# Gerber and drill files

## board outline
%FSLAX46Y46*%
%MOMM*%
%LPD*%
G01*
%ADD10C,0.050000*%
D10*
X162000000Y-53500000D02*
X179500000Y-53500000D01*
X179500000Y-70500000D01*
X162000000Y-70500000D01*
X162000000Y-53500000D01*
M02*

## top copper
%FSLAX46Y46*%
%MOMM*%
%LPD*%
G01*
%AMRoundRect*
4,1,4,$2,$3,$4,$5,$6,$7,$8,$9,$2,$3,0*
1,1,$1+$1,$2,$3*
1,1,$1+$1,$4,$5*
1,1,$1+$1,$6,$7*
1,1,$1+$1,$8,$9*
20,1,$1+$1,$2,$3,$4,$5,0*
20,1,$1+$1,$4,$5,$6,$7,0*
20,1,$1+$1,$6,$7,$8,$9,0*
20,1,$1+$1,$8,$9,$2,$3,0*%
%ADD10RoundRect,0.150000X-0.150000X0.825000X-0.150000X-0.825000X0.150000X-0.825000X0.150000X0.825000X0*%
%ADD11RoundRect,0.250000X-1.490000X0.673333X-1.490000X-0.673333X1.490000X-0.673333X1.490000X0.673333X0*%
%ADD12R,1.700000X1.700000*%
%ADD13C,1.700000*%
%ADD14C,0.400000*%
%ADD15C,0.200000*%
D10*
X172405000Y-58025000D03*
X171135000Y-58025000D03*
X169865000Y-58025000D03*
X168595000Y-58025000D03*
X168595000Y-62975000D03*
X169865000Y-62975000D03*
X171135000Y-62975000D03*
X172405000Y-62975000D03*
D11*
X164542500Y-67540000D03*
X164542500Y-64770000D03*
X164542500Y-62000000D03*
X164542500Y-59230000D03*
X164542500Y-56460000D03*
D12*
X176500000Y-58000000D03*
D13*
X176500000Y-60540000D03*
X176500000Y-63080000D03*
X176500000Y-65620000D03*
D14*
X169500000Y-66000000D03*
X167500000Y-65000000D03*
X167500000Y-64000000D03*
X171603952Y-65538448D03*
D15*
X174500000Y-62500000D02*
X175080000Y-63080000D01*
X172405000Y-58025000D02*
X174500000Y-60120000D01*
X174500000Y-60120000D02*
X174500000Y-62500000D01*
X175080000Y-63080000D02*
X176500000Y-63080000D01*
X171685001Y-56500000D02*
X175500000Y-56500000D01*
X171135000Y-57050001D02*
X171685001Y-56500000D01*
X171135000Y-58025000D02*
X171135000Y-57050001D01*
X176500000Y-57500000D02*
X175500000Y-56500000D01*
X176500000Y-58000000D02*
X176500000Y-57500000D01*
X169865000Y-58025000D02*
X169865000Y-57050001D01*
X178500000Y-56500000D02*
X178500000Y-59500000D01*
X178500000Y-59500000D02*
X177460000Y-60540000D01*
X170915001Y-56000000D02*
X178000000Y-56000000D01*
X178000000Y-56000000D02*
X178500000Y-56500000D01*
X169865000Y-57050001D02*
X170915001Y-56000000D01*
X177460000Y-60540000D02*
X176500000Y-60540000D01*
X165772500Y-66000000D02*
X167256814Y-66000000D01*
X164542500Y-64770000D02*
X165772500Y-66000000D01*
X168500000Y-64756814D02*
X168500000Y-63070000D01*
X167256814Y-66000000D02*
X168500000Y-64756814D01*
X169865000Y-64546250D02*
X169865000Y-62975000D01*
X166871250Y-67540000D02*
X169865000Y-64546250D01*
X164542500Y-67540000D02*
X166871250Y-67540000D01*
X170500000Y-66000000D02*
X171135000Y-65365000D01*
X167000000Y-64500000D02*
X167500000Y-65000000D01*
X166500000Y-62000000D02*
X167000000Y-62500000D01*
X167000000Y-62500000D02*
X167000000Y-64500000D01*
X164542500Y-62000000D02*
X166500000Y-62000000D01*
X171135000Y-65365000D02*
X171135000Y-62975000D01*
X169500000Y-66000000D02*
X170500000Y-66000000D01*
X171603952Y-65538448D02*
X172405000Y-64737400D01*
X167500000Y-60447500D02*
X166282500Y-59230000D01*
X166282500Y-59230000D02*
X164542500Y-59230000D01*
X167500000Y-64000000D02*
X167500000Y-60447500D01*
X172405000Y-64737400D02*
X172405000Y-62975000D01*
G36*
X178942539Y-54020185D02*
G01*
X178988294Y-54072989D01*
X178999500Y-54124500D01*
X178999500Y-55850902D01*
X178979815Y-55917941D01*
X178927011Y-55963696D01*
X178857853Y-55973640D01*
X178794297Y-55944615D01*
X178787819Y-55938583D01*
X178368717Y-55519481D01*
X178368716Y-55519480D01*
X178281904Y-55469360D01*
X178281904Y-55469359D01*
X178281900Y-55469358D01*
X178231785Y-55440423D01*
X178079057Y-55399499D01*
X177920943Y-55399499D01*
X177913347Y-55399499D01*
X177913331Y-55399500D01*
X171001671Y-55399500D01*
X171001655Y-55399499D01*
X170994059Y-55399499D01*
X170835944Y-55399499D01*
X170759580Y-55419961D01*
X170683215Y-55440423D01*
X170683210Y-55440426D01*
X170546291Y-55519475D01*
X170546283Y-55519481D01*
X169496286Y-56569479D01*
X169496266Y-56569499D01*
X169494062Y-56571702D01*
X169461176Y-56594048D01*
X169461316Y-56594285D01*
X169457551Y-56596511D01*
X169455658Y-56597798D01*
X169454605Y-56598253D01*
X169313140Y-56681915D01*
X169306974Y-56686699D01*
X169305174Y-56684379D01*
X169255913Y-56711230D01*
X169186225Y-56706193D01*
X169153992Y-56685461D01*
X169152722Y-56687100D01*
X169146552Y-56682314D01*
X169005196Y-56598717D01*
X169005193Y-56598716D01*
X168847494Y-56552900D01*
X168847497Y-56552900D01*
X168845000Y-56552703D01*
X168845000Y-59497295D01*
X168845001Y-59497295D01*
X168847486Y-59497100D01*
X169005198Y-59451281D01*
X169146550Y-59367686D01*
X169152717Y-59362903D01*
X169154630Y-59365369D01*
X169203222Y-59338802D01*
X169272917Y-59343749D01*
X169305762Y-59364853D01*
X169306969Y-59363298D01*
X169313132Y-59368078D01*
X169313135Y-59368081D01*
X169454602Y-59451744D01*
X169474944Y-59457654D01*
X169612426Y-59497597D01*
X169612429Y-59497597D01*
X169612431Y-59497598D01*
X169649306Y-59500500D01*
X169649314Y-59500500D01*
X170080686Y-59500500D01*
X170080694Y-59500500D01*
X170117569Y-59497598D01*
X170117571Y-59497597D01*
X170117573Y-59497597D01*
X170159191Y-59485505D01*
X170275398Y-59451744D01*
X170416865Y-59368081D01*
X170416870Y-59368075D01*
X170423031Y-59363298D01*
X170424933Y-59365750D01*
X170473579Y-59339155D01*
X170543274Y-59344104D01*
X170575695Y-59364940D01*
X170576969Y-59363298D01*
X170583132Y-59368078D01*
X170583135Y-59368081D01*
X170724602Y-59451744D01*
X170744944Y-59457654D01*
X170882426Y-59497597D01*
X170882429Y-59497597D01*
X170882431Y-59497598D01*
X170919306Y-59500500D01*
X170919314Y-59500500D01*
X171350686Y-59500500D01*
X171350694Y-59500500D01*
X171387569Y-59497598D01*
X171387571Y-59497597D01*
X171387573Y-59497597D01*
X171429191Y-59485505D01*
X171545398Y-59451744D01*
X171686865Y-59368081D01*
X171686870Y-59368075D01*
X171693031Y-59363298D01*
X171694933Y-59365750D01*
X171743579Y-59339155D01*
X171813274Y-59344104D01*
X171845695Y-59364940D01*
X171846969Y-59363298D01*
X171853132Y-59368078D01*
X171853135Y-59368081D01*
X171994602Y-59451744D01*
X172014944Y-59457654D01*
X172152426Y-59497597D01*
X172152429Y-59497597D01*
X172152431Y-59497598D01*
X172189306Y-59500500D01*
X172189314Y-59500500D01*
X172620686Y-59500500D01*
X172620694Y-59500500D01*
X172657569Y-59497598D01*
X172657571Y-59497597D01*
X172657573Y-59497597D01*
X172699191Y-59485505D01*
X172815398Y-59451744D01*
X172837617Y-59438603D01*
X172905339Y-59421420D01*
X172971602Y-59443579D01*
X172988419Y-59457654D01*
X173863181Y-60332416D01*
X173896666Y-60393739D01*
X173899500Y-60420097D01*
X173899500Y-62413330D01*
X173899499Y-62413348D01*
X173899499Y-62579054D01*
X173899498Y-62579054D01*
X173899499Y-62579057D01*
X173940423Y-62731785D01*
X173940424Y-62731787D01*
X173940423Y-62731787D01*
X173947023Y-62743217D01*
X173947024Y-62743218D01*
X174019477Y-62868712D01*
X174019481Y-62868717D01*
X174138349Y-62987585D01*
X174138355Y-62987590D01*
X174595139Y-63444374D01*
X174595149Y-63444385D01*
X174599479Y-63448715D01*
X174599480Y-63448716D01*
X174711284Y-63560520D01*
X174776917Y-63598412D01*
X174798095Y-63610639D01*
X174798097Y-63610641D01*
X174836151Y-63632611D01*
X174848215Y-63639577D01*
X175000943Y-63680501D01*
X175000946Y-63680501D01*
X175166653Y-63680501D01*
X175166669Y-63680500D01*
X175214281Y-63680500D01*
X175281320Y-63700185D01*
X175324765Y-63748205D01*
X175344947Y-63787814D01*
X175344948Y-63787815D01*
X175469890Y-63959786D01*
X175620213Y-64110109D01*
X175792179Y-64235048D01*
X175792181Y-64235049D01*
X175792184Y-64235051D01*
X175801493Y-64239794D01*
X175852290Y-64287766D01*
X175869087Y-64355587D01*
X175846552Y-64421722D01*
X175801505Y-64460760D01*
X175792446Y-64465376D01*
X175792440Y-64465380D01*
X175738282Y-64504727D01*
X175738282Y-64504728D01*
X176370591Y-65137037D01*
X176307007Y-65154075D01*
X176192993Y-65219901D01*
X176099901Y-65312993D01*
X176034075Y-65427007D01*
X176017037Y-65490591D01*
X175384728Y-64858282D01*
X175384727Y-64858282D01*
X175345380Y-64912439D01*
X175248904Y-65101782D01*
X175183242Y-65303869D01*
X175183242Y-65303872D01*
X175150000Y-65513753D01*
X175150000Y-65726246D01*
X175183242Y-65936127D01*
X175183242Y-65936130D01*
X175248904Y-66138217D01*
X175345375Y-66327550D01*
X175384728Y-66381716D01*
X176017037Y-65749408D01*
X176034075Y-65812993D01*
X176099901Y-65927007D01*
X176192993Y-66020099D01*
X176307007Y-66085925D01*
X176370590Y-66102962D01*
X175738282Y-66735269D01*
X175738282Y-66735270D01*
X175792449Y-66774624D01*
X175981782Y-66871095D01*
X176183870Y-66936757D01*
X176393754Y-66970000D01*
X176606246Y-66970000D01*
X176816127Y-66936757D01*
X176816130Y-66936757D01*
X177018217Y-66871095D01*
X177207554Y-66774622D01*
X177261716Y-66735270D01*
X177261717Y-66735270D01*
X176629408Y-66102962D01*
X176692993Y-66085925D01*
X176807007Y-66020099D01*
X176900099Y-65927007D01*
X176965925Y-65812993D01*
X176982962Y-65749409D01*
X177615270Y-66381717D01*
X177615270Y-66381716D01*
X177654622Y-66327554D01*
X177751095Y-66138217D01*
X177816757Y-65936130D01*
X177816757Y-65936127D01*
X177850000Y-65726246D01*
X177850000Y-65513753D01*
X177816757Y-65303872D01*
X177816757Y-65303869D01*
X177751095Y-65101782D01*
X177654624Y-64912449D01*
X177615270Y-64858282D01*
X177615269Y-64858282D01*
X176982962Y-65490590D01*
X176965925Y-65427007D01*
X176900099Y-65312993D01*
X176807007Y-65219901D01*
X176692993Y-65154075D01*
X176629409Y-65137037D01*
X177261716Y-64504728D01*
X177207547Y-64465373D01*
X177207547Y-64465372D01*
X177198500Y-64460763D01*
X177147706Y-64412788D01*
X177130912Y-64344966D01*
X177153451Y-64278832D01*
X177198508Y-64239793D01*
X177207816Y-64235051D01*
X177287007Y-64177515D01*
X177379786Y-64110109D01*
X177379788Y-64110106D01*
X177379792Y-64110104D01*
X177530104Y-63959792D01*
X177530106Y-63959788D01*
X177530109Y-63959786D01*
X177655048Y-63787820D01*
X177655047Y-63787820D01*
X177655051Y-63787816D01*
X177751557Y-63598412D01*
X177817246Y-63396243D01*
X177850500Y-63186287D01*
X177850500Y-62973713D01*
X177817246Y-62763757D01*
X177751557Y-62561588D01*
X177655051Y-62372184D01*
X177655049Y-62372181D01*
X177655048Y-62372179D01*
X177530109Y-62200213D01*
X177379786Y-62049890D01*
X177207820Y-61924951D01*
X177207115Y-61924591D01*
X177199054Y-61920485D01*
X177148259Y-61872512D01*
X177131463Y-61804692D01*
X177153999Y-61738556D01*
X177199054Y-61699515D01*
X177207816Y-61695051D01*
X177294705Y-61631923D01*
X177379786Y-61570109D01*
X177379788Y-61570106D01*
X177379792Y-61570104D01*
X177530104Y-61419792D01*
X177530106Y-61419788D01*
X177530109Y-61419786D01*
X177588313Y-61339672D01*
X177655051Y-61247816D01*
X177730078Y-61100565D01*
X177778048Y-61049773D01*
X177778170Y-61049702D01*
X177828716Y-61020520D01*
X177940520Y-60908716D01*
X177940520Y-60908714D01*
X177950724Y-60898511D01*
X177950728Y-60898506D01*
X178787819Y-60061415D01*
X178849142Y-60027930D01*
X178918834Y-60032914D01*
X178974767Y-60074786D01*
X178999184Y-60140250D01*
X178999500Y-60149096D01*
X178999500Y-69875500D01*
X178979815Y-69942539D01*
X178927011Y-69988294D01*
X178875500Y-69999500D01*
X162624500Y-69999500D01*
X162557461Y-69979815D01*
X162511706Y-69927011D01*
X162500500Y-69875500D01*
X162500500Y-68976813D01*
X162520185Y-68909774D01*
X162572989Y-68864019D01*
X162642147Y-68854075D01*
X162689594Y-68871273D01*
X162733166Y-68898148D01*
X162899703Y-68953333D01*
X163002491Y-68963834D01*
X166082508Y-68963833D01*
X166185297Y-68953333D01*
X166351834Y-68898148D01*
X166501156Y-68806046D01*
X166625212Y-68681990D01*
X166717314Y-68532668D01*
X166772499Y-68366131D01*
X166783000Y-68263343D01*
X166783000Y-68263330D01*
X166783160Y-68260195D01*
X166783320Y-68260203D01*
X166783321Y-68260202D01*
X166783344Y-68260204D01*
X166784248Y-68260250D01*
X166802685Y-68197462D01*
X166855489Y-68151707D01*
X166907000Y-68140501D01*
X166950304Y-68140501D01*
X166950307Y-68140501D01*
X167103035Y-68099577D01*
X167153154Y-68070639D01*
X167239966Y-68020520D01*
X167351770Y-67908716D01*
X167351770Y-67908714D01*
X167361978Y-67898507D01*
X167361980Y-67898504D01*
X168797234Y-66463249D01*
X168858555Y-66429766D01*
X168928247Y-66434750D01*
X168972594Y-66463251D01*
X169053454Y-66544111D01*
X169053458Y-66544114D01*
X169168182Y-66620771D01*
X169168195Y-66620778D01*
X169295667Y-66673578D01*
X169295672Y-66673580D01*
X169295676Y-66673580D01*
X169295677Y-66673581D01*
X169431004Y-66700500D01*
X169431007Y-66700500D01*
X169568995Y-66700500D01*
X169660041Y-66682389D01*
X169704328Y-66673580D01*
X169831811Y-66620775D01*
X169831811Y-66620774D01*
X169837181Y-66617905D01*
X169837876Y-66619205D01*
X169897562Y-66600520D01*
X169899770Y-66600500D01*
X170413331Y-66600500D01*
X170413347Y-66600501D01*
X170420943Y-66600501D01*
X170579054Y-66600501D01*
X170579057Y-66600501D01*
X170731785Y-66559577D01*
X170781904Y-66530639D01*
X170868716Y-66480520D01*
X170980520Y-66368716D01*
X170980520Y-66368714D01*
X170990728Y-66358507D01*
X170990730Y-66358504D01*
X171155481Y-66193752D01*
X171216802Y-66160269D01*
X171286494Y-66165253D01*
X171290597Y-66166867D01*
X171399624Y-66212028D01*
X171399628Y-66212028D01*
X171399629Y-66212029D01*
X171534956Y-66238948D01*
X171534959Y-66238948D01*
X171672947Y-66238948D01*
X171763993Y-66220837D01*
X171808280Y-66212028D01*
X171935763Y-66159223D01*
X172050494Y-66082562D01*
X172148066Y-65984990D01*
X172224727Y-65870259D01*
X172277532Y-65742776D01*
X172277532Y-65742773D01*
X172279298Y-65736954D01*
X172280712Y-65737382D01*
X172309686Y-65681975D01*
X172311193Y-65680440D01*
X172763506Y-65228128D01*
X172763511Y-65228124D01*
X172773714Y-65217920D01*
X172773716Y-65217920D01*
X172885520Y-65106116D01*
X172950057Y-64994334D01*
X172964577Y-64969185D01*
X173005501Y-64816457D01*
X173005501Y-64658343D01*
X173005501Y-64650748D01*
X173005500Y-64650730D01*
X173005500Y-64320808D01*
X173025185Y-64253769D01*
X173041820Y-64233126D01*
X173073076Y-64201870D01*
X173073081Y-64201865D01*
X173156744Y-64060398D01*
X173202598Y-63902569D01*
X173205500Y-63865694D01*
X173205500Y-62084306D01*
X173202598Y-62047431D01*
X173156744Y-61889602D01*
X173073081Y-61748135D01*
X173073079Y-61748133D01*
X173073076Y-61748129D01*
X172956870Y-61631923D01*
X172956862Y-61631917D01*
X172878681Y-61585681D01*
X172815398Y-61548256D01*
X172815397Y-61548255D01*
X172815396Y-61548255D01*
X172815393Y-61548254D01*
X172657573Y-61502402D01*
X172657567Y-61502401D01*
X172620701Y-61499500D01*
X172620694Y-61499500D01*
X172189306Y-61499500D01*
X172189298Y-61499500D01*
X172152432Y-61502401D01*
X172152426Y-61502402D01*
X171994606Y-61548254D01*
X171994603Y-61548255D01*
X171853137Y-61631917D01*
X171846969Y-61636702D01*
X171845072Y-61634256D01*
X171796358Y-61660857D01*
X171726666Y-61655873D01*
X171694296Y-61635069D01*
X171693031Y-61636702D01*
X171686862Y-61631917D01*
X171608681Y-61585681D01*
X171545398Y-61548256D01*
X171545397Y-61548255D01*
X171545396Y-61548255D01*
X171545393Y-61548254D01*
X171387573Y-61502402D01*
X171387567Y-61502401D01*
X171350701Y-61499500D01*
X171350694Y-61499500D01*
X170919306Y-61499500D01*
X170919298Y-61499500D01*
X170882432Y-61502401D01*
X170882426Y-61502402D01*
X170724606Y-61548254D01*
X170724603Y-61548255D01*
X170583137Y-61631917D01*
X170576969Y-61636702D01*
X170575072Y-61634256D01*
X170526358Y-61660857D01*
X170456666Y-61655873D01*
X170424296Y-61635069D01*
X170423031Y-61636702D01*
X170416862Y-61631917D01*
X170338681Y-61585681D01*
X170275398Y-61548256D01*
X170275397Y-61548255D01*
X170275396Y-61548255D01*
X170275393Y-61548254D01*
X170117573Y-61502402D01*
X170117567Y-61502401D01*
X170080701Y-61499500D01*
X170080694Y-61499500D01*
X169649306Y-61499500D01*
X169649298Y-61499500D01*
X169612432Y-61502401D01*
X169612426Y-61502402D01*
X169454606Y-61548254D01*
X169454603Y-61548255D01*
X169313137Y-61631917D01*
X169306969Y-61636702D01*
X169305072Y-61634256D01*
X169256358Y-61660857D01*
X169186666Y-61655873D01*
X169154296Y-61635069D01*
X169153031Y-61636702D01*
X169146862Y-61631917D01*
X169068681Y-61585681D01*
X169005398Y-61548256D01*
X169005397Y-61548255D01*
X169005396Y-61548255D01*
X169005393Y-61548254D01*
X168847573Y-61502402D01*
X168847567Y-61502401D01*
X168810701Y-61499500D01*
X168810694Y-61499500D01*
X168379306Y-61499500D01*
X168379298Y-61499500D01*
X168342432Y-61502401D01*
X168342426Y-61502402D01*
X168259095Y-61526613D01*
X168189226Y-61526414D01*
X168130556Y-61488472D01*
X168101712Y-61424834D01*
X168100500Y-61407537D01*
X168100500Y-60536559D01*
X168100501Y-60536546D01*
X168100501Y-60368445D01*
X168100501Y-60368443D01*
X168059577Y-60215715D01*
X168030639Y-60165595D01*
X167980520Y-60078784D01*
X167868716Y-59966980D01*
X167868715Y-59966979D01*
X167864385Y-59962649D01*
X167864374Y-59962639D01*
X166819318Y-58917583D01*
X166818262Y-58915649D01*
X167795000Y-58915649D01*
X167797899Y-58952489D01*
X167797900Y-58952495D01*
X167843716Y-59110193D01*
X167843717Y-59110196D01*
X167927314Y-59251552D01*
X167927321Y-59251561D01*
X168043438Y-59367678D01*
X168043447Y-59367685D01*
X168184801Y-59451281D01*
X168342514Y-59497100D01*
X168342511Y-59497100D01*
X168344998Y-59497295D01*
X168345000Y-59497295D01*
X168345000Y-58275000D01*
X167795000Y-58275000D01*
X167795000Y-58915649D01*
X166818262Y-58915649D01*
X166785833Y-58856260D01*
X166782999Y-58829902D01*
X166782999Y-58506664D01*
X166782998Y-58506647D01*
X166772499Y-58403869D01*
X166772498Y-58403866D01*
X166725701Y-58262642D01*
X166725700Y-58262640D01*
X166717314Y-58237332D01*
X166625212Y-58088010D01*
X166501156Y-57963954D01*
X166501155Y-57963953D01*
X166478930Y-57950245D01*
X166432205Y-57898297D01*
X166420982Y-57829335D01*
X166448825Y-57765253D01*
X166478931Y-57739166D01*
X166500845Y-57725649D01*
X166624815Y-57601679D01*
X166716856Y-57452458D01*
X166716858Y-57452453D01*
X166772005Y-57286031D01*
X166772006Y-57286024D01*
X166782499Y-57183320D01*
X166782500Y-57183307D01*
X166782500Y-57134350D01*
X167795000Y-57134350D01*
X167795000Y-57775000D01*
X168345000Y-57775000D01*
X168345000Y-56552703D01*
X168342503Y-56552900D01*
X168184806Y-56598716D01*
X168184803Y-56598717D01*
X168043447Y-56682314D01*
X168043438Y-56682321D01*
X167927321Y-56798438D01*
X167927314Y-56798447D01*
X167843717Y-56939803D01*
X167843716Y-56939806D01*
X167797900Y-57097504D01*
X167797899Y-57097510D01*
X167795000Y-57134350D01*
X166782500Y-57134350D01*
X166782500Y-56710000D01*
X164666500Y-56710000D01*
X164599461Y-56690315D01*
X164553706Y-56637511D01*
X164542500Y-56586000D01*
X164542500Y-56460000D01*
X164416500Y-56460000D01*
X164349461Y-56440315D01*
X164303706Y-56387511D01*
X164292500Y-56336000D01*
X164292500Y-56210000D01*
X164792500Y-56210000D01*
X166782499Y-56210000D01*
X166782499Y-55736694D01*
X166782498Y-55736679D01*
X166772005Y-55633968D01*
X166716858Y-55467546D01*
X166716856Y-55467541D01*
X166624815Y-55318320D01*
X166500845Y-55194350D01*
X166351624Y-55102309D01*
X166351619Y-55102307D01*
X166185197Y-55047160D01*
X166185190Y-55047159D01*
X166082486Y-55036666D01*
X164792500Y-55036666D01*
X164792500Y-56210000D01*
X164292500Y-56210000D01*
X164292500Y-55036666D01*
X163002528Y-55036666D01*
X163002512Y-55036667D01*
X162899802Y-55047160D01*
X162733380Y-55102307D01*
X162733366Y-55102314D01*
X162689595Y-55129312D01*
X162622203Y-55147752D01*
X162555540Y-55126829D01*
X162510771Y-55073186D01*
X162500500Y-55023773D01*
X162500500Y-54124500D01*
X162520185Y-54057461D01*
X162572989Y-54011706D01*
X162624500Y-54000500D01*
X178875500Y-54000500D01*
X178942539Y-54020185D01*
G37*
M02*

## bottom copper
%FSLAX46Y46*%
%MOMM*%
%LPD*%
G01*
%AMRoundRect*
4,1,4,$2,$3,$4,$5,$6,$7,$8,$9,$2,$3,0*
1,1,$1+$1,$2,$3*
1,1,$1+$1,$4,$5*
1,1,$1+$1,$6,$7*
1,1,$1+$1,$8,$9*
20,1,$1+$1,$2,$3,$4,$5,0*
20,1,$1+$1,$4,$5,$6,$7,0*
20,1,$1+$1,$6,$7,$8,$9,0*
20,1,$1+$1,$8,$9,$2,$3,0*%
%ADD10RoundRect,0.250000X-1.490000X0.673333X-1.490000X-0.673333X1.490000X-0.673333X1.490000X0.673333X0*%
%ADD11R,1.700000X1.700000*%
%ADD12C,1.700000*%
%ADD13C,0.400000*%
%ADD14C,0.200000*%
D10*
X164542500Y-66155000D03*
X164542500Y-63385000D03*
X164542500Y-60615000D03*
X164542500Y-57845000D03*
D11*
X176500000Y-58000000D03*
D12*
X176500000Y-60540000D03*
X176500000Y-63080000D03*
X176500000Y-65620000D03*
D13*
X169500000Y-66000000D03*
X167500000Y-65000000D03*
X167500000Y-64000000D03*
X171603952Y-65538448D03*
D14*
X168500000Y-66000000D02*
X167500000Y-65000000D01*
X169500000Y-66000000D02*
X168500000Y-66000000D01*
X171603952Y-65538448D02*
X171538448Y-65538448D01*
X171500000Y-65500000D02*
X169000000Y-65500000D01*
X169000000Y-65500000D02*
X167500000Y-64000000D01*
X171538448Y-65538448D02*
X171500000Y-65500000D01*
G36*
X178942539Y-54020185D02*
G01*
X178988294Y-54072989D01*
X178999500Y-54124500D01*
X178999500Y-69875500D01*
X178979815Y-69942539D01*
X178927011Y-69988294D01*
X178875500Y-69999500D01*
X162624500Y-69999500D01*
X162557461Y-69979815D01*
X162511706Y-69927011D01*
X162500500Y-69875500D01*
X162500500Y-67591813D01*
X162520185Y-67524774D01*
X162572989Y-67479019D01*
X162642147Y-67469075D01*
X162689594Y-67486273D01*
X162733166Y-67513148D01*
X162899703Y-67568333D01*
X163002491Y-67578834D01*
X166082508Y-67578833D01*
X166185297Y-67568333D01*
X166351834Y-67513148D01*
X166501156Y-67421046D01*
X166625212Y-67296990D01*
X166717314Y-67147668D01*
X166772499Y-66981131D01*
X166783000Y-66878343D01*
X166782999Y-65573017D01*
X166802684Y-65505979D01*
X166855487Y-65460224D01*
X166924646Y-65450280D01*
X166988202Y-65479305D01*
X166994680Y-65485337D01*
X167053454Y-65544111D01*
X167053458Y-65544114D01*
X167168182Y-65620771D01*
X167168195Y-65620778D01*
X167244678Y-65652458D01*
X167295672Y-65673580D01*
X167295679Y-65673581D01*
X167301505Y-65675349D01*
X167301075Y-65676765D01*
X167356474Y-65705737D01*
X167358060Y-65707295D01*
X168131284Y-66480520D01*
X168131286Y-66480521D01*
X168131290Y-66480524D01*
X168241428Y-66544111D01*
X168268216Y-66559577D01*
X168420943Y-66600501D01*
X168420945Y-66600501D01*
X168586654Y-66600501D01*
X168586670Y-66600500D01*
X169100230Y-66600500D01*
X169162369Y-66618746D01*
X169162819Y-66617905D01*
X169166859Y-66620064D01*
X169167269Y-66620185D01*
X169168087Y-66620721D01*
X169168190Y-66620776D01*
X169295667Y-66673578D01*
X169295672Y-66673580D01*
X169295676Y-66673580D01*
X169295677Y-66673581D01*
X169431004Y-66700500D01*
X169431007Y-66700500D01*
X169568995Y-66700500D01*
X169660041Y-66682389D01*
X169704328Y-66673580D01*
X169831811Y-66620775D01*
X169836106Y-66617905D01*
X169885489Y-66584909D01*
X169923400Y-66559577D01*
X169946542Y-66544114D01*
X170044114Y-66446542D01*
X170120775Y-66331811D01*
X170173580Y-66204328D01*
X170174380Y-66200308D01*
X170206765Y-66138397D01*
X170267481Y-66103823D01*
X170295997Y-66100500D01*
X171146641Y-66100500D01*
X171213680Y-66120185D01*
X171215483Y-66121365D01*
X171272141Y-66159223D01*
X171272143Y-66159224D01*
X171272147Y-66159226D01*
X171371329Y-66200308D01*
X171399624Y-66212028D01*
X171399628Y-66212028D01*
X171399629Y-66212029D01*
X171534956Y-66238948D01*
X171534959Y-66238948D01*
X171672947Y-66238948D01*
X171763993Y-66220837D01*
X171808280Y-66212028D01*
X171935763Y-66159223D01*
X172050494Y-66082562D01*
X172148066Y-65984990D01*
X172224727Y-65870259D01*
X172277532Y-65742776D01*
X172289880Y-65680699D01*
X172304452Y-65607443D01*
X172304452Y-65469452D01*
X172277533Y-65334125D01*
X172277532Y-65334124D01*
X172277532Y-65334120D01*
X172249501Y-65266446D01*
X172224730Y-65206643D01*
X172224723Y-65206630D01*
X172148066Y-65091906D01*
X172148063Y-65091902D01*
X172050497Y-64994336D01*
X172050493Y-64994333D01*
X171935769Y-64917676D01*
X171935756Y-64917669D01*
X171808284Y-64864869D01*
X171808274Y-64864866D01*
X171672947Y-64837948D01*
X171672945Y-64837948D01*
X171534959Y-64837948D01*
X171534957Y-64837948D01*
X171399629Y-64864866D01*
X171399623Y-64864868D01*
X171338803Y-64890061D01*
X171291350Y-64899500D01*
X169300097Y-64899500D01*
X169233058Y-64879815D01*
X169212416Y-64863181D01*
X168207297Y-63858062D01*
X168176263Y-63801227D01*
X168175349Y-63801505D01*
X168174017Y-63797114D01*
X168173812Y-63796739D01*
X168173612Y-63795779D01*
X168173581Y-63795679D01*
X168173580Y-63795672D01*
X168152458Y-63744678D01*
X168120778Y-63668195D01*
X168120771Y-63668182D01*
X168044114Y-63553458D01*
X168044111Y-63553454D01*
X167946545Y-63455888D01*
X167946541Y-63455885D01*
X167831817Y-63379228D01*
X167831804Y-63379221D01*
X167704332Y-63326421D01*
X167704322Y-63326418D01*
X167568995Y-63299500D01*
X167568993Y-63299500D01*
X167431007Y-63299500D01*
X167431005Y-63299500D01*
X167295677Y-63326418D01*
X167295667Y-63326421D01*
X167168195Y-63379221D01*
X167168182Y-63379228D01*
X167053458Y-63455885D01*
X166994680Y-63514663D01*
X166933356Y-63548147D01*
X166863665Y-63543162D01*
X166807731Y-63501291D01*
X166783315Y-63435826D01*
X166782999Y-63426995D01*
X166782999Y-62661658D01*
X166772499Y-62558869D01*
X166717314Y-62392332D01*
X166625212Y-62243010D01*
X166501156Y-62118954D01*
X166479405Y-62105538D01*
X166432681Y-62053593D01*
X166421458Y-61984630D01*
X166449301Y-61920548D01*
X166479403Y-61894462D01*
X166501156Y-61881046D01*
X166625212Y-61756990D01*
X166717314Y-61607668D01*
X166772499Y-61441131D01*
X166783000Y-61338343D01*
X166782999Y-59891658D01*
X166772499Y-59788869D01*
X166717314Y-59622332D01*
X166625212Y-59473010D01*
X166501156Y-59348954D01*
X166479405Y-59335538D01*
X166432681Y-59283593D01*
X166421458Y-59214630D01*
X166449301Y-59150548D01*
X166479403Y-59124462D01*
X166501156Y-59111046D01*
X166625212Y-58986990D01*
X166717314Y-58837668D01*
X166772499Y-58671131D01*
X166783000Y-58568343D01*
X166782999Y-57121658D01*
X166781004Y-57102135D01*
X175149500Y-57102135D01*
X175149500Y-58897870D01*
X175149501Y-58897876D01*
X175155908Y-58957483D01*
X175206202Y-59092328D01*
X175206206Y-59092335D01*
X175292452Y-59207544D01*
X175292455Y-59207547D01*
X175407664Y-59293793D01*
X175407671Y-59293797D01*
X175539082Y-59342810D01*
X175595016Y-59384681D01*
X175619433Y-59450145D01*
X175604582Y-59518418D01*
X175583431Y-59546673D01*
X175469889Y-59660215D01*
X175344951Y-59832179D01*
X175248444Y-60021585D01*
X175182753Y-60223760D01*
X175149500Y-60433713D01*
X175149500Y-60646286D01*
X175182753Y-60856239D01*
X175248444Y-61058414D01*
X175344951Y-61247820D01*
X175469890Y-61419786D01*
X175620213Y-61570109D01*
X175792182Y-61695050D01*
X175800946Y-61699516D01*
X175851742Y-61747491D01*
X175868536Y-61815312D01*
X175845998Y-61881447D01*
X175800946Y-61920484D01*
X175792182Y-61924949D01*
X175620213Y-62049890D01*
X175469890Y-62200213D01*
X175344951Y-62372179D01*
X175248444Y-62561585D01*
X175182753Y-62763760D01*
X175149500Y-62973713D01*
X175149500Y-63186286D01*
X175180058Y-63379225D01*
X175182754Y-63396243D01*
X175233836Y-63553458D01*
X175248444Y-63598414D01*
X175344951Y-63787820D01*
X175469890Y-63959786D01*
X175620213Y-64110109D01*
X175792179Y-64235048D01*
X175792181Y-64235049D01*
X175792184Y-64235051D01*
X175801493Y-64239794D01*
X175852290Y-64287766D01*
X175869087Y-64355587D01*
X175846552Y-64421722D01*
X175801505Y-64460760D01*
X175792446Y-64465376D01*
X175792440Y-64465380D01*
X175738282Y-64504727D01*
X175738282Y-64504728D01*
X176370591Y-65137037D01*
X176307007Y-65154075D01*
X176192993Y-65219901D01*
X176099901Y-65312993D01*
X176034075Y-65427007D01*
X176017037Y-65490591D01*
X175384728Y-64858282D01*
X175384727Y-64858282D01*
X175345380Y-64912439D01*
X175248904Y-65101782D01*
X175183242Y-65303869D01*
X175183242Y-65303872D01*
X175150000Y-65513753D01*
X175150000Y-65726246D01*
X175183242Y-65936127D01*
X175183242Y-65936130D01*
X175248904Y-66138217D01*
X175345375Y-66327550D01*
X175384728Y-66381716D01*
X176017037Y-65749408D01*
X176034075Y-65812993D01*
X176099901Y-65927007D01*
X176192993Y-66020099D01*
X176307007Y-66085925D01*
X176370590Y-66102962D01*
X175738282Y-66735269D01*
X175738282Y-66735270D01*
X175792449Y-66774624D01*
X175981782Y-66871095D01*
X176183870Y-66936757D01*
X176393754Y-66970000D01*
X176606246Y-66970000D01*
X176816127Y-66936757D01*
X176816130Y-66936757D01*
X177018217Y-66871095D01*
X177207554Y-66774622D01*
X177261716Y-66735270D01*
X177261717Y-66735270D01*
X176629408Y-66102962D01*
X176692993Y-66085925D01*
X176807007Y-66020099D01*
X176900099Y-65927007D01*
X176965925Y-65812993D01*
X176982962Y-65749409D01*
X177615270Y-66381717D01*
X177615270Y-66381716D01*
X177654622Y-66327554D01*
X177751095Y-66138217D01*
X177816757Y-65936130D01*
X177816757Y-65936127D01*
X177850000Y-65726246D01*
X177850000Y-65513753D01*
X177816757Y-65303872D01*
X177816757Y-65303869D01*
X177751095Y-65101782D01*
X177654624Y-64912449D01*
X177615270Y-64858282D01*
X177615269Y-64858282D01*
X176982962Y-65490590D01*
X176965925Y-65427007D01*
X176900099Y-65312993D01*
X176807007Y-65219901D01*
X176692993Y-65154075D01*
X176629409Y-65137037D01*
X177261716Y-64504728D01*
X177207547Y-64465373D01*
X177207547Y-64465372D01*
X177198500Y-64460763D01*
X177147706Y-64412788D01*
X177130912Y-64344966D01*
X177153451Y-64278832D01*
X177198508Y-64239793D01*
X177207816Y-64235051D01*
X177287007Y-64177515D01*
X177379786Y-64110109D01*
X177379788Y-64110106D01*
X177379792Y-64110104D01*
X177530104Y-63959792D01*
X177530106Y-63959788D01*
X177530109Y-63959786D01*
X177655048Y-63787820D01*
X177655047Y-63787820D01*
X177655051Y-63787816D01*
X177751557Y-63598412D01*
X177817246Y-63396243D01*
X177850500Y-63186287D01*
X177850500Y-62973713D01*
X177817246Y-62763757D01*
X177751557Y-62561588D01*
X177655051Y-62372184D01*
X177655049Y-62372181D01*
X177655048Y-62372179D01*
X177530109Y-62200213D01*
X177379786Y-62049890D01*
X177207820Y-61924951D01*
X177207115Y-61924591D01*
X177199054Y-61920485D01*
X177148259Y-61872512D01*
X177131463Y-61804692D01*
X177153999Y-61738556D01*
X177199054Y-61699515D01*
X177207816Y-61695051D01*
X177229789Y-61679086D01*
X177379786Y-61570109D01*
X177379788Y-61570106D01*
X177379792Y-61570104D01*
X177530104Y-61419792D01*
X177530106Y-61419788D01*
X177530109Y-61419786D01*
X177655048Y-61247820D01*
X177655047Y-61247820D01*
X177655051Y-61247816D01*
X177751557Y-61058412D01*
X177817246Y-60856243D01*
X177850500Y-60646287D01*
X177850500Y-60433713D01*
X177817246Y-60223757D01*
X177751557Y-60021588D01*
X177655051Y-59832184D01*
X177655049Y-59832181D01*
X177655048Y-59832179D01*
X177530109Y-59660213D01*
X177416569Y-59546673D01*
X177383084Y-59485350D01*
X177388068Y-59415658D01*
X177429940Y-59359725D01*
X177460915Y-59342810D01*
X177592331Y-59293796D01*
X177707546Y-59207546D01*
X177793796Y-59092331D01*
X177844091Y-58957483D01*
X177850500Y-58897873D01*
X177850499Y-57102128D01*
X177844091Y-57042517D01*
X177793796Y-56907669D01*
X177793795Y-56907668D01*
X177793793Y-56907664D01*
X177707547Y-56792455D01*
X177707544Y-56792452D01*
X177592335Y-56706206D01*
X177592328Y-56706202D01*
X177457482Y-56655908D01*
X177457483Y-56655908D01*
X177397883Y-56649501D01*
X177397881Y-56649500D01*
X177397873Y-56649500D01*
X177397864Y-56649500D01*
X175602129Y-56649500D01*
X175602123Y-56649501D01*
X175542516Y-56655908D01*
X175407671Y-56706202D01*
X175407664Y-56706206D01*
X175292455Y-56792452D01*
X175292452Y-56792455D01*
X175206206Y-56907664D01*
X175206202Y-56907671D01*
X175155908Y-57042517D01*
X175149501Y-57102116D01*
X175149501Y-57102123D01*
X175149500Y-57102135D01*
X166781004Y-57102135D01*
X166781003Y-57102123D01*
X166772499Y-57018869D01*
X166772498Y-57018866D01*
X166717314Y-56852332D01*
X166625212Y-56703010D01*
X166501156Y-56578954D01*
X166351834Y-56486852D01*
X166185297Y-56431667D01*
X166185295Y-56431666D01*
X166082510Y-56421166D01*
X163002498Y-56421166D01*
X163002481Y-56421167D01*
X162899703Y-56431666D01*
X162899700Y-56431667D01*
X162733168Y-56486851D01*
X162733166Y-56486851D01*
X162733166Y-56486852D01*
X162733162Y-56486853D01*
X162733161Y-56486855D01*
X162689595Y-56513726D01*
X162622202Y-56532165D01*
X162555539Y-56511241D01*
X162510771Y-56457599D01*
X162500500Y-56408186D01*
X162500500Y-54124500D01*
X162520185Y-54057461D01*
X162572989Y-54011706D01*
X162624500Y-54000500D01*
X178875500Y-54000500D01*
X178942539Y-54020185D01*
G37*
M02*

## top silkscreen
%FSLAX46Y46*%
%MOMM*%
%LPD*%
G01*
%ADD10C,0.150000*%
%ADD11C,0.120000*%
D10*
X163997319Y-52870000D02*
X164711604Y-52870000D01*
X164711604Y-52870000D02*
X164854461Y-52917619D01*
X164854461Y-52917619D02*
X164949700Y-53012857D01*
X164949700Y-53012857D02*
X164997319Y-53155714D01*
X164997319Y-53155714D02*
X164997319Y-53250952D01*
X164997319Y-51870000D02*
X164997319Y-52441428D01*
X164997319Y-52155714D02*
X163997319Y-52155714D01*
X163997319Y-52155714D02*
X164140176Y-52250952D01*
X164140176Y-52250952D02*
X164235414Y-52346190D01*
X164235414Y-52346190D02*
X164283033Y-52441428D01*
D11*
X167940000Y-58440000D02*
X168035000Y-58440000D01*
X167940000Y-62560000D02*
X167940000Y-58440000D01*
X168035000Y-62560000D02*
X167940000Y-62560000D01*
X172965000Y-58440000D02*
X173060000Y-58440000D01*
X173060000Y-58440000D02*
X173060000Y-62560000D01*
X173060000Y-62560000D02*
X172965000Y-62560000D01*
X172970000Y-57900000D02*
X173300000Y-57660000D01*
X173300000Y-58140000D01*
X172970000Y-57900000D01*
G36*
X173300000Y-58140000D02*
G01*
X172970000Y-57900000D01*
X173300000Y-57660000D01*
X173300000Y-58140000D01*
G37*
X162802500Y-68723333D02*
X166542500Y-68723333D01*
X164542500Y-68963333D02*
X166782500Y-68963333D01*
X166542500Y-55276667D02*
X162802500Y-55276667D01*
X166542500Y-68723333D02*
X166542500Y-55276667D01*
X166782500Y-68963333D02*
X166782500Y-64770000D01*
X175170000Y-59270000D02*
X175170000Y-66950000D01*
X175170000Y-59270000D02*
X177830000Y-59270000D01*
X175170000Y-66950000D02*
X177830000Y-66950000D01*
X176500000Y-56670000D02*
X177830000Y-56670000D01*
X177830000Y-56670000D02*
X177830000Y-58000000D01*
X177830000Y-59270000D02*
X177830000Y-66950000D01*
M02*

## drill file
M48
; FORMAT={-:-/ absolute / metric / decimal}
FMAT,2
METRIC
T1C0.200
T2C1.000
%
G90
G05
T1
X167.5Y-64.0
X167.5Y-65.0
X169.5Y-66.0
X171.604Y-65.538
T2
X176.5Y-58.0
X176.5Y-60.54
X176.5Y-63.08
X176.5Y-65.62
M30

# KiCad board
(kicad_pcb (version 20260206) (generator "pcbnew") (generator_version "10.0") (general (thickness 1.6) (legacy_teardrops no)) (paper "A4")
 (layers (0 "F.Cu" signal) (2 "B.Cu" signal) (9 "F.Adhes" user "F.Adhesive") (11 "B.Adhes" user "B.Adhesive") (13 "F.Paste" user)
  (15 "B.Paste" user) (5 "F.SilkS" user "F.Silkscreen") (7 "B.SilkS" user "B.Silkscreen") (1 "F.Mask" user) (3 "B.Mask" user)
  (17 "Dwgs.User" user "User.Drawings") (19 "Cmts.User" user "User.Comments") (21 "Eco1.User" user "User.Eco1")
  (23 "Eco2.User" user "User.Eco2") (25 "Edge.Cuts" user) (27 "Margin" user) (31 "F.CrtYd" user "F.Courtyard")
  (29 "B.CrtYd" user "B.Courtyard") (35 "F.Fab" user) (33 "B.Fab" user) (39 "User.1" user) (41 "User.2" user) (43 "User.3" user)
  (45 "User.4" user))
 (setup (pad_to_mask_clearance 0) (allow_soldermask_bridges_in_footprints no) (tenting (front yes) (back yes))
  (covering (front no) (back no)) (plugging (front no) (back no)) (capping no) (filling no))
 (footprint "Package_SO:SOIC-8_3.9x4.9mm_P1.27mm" (layer "F.Cu") (at 170.5 60.5 -90)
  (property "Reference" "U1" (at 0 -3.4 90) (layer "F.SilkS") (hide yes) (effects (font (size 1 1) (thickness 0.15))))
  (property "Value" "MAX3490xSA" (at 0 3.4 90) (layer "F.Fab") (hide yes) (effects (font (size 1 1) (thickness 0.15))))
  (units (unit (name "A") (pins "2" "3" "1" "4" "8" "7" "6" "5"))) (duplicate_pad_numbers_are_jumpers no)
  (fp_line (start -2.06 2.56) (end -2.06 2.465) (stroke (width 0.12) (type solid)) (layer "F.SilkS"))
  (fp_line (start 2.06 2.56) (end -2.06 2.56) (stroke (width 0.12) (type solid)) (layer "F.SilkS"))
  (fp_line (start 2.06 2.465) (end 2.06 2.56) (stroke (width 0.12) (type solid)) (layer "F.SilkS"))
  (fp_line (start -2.06 -2.465) (end -2.06 -2.56) (stroke (width 0.12) (type solid)) (layer "F.SilkS"))
  (fp_line (start -2.06 -2.56) (end 2.06 -2.56) (stroke (width 0.12) (type solid)) (layer "F.SilkS"))
  (fp_line (start 2.06 -2.56) (end 2.06 -2.465) (stroke (width 0.12) (type solid)) (layer "F.SilkS"))
  (fp_poly (pts (xy -2.6 -2.47) (xy -2.84 -2.8) (xy -2.36 -2.8)) (stroke (width 0.12) (type solid)) (fill yes) (layer "F.SilkS"))
  (pad "1" smd roundrect (at -2.475 -1.905 270) (size 1.95 0.6) (layers "F.Cu" "F.Mask" "F.Paste") (roundrect_rratio 0.25) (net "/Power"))
  (pad "2" smd roundrect (at -2.475 -0.635 270) (size 1.95 0.6) (layers "F.Cu" "F.Mask" "F.Paste") (roundrect_rratio 0.25) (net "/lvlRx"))
  (pad "3" smd roundrect (at -2.475 0.635 270) (size 1.95 0.6) (layers "F.Cu" "F.Mask" "F.Paste") (roundrect_rratio 0.25) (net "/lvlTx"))
  (pad "4" smd roundrect (at -2.475 1.905 270) (size 1.95 0.6) (layers "F.Cu" "F.Mask" "F.Paste") (roundrect_rratio 0.25) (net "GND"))
  (pad "5" smd roundrect (at 2.475 1.905 270) (size 1.95 0.6) (layers "F.Cu" "F.Mask" "F.Paste") (roundrect_rratio 0.25) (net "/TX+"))
  (pad "6" smd roundrect (at 2.475 0.635 270) (size 1.95 0.6) (layers "F.Cu" "F.Mask" "F.Paste") (roundrect_rratio 0.25) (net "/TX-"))
  (pad "7" smd roundrect (at 2.475 -0.635 270) (size 1.95 0.6) (layers "F.Cu" "F.Mask" "F.Paste") (roundrect_rratio 0.25) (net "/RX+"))
  (pad "8" smd roundrect (at 2.475 -1.905 270) (size 1.95 0.6) (layers "F.Cu" "F.Mask" "F.Paste") (roundrect_rratio 0.25) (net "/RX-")))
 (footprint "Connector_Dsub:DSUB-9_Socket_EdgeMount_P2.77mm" (layer "F.Cu") (at 164.5425 62 -90)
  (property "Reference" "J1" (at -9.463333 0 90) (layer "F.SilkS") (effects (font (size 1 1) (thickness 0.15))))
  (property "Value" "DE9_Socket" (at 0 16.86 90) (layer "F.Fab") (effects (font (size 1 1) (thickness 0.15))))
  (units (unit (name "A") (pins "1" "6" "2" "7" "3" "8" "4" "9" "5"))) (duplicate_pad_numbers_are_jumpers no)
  (fp_line (start 6.723333 1.74) (end 6.723333 -2) (stroke (width 0.12) (type solid)) (layer "F.SilkS"))
  (fp_line (start 6.963333 0) (end 6.963333 -2.24) (stroke (width 0.12) (type solid)) (layer "F.SilkS"))
  (fp_line (start -6.723333 -2) (end -6.723333 1.74) (stroke (width 0.12) (type solid)) (layer "F.SilkS"))
  (fp_line (start 6.723333 -2) (end -6.723333 -2) (stroke (width 0.12) (type solid)) (layer "F.SilkS"))
  (fp_line (start 6.963333 -2.24) (end 2.77 -2.24) (stroke (width 0.12) (type solid)) (layer "F.SilkS"))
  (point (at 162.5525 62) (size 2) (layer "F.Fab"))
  (pad "1" smd roundrect (at 5.54 0 270) (size 1.846667 3.48) (layers "F.Cu" "F.Mask" "F.Paste") (roundrect_rratio 0.135379) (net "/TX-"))
  (pad "2" smd roundrect (at 2.77 0 270) (size 1.846667 3.48) (layers "F.Cu" "F.Mask" "F.Paste") (roundrect_rratio 0.135379) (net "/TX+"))
  (pad "3" smd roundrect (at 0 0 270) (size 1.846667 3.48) (layers "F.Cu" "F.Mask" "F.Paste") (roundrect_rratio 0.135379) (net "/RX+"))
  (pad "4" smd roundrect (at -2.77 0 270) (size 1.846667 3.48) (layers "F.Cu" "F.Mask" "F.Paste") (roundrect_rratio 0.135379) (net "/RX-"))
  (pad "5" smd roundrect (at -5.54 0 270) (size 1.846667 3.48) (layers "F.Cu" "F.Mask" "F.Paste") (roundrect_rratio 0.135379) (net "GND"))
  (pad "6" smd roundrect (at 4.155 0 270) (size 1.846667 3.48) (layers "B.Cu" "B.Mask" "B.Paste") (roundrect_rratio 0.135379)
   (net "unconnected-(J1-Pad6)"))
  (pad "7" smd roundrect (at 1.385 0 270) (size 1.846667 3.48) (layers "B.Cu" "B.Mask" "B.Paste") (roundrect_rratio 0.135379)
   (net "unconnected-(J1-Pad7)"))
  (pad "8" smd roundrect (at -1.385 0 270) (size 1.846667 3.48) (layers "B.Cu" "B.Mask" "B.Paste") (roundrect_rratio 0.135379)
   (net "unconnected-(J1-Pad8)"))
  (pad "9" smd roundrect (at -4.155 0 270) (size 1.846667 3.48) (layers "B.Cu" "B.Mask" "B.Paste") (roundrect_rratio 0.135379)
   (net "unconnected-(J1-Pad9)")))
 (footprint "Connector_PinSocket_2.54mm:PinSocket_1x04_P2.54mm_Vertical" (layer "F.Cu") (at 176.5 58)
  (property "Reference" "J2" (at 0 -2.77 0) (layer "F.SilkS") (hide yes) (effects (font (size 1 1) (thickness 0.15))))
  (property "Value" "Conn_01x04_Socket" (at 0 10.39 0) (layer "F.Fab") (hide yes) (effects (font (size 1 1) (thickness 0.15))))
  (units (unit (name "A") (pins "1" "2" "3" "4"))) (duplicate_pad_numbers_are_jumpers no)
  (fp_line (start -1.33 1.27) (end -1.33 8.95) (stroke (width 0.12) (type solid)) (layer "F.SilkS"))
  (fp_line (start -1.33 1.27) (end 1.33 1.27) (stroke (width 0.12) (type solid)) (layer "F.SilkS"))
  (fp_line (start -1.33 8.95) (end 1.33 8.95) (stroke (width 0.12) (type solid)) (layer "F.SilkS"))
  (fp_line (start 0 -1.33) (end 1.33 -1.33) (stroke (width 0.12) (type solid)) (layer "F.SilkS"))
  (fp_line (start 1.33 -1.33) (end 1.33 0) (stroke (width 0.12) (type solid)) (layer "F.SilkS"))
  (fp_line (start 1.33 1.27) (end 1.33 8.95) (stroke (width 0.12) (type solid)) (layer "F.SilkS"))
  (pad "1" thru_hole rect (at 0 0) (size 1.7 1.7) (drill 1) (layers "*.Cu" "*.Mask") (remove_unused_layers no) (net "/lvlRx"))
  (pad "2" thru_hole circle (at 0 2.54) (size 1.7 1.7) (drill 1) (layers "*.Cu" "*.Mask") (remove_unused_layers no) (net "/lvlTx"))
  (pad "3" thru_hole circle (at 0 5.08) (size 1.7 1.7) (drill 1) (layers "*.Cu" "*.Mask") (remove_unused_layers no) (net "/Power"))
  (pad "4" thru_hole circle (at 0 7.62) (size 1.7 1.7) (drill 1) (layers "*.Cu" "*.Mask") (remove_unused_layers no) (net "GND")))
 (gr_rect (start 162 53.5) (end 179.5 70.5) (stroke (width 0.05) (type default)) (fill no) (layer "Edge.Cuts"))
 (segment (start 174.5 62.5) (end 175.08 63.08) (width 0.2) (layer "F.Cu") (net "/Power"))
 (segment (start 172.405 58.025) (end 174.5 60.12) (width 0.2) (layer "F.Cu") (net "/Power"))
 (segment (start 174.5 60.12) (end 174.5 62.5) (width 0.2) (layer "F.Cu") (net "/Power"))
 (segment (start 175.08 63.08) (end 176.5 63.08) (width 0.2) (layer "F.Cu") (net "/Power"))
 (segment (start 171.685001 56.5) (end 175.5 56.5) (width 0.2) (layer "F.Cu") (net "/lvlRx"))
 (segment (start 171.135 57.050001) (end 171.685001 56.5) (width 0.2) (layer "F.Cu") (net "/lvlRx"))
 (segment (start 171.135 58.025) (end 171.135 57.050001) (width 0.2) (layer "F.Cu") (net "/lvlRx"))
 (segment (start 176.5 57.5) (end 175.5 56.5) (width 0.2) (layer "F.Cu") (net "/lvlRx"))
 (segment (start 176.5 58) (end 176.5 57.5) (width 0.2) (layer "F.Cu") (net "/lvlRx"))
 (segment (start 169.865 58.025) (end 169.865 57.050001) (width 0.2) (layer "F.Cu") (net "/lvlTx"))
 (segment (start 178.5 56.5) (end 178.5 59.5) (width 0.2) (layer "F.Cu") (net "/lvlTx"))
 (segment (start 178.5 59.5) (end 177.46 60.54) (width 0.2) (layer "F.Cu") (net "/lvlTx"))
 (segment (start 170.915001 56) (end 178 56) (width 0.2) (layer "F.Cu") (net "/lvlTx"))
 (segment (start 178 56) (end 178.5 56.5) (width 0.2) (layer "F.Cu") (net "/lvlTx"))
 (segment (start 169.865 57.050001) (end 170.915001 56) (width 0.2) (layer "F.Cu") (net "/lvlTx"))
 (segment (start 177.46 60.54) (end 176.5 60.54) (width 0.2) (layer "F.Cu") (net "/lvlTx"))
 (segment (start 165.7725 66) (end 167.256814 66) (width 0.2) (layer "F.Cu") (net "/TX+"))
 (segment (start 164.5425 64.77) (end 165.7725 66) (width 0.2) (layer "F.Cu") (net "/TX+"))
 (segment (start 168.5 64.756814) (end 168.5 63.07) (width 0.2) (layer "F.Cu") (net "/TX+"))
 (segment (start 167.256814 66) (end 168.5 64.756814) (width 0.2) (layer "F.Cu") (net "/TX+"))
 (segment (start 169.865 64.54625) (end 169.865 62.975) (width 0.2) (layer "F.Cu") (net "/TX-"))
 (segment (start 166.87125 67.54) (end 169.865 64.54625) (width 0.2) (layer "F.Cu") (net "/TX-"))
 (segment (start 164.5425 67.54) (end 166.87125 67.54) (width 0.2) (layer "F.Cu") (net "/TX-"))
 (segment (start 170.5 66) (end 171.135 65.365) (width 0.2) (layer "F.Cu") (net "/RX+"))
 (segment (start 167 64.5) (end 167.5 65) (width 0.2) (layer "F.Cu") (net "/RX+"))
 (segment (start 166.5 62) (end 167 62.5) (width 0.2) (layer "F.Cu") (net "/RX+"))
 (segment (start 167 62.5) (end 167 64.5) (width 0.2) (layer "F.Cu") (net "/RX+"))
 (segment (start 164.5425 62) (end 166.5 62) (width 0.2) (layer "F.Cu") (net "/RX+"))
 (segment (start 171.135 65.365) (end 171.135 62.975) (width 0.2) (layer "F.Cu") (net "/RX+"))
 (segment (start 169.5 66) (end 170.5 66) (width 0.2) (layer "F.Cu") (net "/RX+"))
 (via (at 169.5 66) (size 0.4) (drill 0.2) (layers "F.Cu" "B.Cu") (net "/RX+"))
 (via (at 167.5 65) (size 0.4) (drill 0.2) (layers "F.Cu" "B.Cu") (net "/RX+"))
 (segment (start 168.5 66) (end 167.5 65) (width 0.2) (layer "B.Cu") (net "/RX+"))
 (segment (start 169.5 66) (end 168.5 66) (width 0.2) (layer "B.Cu") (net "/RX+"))
 (segment (start 171.603952 65.538448) (end 172.405 64.7374) (width 0.2) (layer "F.Cu") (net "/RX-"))
 (segment (start 167.5 60.4475) (end 166.2825 59.23) (width 0.2) (layer "F.Cu") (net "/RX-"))
 (segment (start 166.2825 59.23) (end 164.5425 59.23) (width 0.2) (layer "F.Cu") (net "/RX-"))
 (segment (start 167.5 64) (end 167.5 60.4475) (width 0.2) (layer "F.Cu") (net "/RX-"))
 (segment (start 172.405 64.7374) (end 172.405 62.975) (width 0.2) (layer "F.Cu") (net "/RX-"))
 (via (at 167.5 64) (size 0.4) (drill 0.2) (layers "F.Cu" "B.Cu") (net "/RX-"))
 (via (at 171.603952 65.538448) (size 0.4) (drill 0.2) (layers "F.Cu" "B.Cu") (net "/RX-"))
 (segment (start 171.603952 65.538448) (end 171.538448 65.538448) (width 0.2) (layer "B.Cu") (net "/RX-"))
 (segment (start 171.5 65.5) (end 169 65.5) (width 0.2) (layer "B.Cu") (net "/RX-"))
 (segment (start 169 65.5) (end 167.5 64) (width 0.2) (layer "B.Cu") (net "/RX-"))
 (segment (start 171.538448 65.538448) (end 171.5 65.5) (width 0.2) (layer "B.Cu") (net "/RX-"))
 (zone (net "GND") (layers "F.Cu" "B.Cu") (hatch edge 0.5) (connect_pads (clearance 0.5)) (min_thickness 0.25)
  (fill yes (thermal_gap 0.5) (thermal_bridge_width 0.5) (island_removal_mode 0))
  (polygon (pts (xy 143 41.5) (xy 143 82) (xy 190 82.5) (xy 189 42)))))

